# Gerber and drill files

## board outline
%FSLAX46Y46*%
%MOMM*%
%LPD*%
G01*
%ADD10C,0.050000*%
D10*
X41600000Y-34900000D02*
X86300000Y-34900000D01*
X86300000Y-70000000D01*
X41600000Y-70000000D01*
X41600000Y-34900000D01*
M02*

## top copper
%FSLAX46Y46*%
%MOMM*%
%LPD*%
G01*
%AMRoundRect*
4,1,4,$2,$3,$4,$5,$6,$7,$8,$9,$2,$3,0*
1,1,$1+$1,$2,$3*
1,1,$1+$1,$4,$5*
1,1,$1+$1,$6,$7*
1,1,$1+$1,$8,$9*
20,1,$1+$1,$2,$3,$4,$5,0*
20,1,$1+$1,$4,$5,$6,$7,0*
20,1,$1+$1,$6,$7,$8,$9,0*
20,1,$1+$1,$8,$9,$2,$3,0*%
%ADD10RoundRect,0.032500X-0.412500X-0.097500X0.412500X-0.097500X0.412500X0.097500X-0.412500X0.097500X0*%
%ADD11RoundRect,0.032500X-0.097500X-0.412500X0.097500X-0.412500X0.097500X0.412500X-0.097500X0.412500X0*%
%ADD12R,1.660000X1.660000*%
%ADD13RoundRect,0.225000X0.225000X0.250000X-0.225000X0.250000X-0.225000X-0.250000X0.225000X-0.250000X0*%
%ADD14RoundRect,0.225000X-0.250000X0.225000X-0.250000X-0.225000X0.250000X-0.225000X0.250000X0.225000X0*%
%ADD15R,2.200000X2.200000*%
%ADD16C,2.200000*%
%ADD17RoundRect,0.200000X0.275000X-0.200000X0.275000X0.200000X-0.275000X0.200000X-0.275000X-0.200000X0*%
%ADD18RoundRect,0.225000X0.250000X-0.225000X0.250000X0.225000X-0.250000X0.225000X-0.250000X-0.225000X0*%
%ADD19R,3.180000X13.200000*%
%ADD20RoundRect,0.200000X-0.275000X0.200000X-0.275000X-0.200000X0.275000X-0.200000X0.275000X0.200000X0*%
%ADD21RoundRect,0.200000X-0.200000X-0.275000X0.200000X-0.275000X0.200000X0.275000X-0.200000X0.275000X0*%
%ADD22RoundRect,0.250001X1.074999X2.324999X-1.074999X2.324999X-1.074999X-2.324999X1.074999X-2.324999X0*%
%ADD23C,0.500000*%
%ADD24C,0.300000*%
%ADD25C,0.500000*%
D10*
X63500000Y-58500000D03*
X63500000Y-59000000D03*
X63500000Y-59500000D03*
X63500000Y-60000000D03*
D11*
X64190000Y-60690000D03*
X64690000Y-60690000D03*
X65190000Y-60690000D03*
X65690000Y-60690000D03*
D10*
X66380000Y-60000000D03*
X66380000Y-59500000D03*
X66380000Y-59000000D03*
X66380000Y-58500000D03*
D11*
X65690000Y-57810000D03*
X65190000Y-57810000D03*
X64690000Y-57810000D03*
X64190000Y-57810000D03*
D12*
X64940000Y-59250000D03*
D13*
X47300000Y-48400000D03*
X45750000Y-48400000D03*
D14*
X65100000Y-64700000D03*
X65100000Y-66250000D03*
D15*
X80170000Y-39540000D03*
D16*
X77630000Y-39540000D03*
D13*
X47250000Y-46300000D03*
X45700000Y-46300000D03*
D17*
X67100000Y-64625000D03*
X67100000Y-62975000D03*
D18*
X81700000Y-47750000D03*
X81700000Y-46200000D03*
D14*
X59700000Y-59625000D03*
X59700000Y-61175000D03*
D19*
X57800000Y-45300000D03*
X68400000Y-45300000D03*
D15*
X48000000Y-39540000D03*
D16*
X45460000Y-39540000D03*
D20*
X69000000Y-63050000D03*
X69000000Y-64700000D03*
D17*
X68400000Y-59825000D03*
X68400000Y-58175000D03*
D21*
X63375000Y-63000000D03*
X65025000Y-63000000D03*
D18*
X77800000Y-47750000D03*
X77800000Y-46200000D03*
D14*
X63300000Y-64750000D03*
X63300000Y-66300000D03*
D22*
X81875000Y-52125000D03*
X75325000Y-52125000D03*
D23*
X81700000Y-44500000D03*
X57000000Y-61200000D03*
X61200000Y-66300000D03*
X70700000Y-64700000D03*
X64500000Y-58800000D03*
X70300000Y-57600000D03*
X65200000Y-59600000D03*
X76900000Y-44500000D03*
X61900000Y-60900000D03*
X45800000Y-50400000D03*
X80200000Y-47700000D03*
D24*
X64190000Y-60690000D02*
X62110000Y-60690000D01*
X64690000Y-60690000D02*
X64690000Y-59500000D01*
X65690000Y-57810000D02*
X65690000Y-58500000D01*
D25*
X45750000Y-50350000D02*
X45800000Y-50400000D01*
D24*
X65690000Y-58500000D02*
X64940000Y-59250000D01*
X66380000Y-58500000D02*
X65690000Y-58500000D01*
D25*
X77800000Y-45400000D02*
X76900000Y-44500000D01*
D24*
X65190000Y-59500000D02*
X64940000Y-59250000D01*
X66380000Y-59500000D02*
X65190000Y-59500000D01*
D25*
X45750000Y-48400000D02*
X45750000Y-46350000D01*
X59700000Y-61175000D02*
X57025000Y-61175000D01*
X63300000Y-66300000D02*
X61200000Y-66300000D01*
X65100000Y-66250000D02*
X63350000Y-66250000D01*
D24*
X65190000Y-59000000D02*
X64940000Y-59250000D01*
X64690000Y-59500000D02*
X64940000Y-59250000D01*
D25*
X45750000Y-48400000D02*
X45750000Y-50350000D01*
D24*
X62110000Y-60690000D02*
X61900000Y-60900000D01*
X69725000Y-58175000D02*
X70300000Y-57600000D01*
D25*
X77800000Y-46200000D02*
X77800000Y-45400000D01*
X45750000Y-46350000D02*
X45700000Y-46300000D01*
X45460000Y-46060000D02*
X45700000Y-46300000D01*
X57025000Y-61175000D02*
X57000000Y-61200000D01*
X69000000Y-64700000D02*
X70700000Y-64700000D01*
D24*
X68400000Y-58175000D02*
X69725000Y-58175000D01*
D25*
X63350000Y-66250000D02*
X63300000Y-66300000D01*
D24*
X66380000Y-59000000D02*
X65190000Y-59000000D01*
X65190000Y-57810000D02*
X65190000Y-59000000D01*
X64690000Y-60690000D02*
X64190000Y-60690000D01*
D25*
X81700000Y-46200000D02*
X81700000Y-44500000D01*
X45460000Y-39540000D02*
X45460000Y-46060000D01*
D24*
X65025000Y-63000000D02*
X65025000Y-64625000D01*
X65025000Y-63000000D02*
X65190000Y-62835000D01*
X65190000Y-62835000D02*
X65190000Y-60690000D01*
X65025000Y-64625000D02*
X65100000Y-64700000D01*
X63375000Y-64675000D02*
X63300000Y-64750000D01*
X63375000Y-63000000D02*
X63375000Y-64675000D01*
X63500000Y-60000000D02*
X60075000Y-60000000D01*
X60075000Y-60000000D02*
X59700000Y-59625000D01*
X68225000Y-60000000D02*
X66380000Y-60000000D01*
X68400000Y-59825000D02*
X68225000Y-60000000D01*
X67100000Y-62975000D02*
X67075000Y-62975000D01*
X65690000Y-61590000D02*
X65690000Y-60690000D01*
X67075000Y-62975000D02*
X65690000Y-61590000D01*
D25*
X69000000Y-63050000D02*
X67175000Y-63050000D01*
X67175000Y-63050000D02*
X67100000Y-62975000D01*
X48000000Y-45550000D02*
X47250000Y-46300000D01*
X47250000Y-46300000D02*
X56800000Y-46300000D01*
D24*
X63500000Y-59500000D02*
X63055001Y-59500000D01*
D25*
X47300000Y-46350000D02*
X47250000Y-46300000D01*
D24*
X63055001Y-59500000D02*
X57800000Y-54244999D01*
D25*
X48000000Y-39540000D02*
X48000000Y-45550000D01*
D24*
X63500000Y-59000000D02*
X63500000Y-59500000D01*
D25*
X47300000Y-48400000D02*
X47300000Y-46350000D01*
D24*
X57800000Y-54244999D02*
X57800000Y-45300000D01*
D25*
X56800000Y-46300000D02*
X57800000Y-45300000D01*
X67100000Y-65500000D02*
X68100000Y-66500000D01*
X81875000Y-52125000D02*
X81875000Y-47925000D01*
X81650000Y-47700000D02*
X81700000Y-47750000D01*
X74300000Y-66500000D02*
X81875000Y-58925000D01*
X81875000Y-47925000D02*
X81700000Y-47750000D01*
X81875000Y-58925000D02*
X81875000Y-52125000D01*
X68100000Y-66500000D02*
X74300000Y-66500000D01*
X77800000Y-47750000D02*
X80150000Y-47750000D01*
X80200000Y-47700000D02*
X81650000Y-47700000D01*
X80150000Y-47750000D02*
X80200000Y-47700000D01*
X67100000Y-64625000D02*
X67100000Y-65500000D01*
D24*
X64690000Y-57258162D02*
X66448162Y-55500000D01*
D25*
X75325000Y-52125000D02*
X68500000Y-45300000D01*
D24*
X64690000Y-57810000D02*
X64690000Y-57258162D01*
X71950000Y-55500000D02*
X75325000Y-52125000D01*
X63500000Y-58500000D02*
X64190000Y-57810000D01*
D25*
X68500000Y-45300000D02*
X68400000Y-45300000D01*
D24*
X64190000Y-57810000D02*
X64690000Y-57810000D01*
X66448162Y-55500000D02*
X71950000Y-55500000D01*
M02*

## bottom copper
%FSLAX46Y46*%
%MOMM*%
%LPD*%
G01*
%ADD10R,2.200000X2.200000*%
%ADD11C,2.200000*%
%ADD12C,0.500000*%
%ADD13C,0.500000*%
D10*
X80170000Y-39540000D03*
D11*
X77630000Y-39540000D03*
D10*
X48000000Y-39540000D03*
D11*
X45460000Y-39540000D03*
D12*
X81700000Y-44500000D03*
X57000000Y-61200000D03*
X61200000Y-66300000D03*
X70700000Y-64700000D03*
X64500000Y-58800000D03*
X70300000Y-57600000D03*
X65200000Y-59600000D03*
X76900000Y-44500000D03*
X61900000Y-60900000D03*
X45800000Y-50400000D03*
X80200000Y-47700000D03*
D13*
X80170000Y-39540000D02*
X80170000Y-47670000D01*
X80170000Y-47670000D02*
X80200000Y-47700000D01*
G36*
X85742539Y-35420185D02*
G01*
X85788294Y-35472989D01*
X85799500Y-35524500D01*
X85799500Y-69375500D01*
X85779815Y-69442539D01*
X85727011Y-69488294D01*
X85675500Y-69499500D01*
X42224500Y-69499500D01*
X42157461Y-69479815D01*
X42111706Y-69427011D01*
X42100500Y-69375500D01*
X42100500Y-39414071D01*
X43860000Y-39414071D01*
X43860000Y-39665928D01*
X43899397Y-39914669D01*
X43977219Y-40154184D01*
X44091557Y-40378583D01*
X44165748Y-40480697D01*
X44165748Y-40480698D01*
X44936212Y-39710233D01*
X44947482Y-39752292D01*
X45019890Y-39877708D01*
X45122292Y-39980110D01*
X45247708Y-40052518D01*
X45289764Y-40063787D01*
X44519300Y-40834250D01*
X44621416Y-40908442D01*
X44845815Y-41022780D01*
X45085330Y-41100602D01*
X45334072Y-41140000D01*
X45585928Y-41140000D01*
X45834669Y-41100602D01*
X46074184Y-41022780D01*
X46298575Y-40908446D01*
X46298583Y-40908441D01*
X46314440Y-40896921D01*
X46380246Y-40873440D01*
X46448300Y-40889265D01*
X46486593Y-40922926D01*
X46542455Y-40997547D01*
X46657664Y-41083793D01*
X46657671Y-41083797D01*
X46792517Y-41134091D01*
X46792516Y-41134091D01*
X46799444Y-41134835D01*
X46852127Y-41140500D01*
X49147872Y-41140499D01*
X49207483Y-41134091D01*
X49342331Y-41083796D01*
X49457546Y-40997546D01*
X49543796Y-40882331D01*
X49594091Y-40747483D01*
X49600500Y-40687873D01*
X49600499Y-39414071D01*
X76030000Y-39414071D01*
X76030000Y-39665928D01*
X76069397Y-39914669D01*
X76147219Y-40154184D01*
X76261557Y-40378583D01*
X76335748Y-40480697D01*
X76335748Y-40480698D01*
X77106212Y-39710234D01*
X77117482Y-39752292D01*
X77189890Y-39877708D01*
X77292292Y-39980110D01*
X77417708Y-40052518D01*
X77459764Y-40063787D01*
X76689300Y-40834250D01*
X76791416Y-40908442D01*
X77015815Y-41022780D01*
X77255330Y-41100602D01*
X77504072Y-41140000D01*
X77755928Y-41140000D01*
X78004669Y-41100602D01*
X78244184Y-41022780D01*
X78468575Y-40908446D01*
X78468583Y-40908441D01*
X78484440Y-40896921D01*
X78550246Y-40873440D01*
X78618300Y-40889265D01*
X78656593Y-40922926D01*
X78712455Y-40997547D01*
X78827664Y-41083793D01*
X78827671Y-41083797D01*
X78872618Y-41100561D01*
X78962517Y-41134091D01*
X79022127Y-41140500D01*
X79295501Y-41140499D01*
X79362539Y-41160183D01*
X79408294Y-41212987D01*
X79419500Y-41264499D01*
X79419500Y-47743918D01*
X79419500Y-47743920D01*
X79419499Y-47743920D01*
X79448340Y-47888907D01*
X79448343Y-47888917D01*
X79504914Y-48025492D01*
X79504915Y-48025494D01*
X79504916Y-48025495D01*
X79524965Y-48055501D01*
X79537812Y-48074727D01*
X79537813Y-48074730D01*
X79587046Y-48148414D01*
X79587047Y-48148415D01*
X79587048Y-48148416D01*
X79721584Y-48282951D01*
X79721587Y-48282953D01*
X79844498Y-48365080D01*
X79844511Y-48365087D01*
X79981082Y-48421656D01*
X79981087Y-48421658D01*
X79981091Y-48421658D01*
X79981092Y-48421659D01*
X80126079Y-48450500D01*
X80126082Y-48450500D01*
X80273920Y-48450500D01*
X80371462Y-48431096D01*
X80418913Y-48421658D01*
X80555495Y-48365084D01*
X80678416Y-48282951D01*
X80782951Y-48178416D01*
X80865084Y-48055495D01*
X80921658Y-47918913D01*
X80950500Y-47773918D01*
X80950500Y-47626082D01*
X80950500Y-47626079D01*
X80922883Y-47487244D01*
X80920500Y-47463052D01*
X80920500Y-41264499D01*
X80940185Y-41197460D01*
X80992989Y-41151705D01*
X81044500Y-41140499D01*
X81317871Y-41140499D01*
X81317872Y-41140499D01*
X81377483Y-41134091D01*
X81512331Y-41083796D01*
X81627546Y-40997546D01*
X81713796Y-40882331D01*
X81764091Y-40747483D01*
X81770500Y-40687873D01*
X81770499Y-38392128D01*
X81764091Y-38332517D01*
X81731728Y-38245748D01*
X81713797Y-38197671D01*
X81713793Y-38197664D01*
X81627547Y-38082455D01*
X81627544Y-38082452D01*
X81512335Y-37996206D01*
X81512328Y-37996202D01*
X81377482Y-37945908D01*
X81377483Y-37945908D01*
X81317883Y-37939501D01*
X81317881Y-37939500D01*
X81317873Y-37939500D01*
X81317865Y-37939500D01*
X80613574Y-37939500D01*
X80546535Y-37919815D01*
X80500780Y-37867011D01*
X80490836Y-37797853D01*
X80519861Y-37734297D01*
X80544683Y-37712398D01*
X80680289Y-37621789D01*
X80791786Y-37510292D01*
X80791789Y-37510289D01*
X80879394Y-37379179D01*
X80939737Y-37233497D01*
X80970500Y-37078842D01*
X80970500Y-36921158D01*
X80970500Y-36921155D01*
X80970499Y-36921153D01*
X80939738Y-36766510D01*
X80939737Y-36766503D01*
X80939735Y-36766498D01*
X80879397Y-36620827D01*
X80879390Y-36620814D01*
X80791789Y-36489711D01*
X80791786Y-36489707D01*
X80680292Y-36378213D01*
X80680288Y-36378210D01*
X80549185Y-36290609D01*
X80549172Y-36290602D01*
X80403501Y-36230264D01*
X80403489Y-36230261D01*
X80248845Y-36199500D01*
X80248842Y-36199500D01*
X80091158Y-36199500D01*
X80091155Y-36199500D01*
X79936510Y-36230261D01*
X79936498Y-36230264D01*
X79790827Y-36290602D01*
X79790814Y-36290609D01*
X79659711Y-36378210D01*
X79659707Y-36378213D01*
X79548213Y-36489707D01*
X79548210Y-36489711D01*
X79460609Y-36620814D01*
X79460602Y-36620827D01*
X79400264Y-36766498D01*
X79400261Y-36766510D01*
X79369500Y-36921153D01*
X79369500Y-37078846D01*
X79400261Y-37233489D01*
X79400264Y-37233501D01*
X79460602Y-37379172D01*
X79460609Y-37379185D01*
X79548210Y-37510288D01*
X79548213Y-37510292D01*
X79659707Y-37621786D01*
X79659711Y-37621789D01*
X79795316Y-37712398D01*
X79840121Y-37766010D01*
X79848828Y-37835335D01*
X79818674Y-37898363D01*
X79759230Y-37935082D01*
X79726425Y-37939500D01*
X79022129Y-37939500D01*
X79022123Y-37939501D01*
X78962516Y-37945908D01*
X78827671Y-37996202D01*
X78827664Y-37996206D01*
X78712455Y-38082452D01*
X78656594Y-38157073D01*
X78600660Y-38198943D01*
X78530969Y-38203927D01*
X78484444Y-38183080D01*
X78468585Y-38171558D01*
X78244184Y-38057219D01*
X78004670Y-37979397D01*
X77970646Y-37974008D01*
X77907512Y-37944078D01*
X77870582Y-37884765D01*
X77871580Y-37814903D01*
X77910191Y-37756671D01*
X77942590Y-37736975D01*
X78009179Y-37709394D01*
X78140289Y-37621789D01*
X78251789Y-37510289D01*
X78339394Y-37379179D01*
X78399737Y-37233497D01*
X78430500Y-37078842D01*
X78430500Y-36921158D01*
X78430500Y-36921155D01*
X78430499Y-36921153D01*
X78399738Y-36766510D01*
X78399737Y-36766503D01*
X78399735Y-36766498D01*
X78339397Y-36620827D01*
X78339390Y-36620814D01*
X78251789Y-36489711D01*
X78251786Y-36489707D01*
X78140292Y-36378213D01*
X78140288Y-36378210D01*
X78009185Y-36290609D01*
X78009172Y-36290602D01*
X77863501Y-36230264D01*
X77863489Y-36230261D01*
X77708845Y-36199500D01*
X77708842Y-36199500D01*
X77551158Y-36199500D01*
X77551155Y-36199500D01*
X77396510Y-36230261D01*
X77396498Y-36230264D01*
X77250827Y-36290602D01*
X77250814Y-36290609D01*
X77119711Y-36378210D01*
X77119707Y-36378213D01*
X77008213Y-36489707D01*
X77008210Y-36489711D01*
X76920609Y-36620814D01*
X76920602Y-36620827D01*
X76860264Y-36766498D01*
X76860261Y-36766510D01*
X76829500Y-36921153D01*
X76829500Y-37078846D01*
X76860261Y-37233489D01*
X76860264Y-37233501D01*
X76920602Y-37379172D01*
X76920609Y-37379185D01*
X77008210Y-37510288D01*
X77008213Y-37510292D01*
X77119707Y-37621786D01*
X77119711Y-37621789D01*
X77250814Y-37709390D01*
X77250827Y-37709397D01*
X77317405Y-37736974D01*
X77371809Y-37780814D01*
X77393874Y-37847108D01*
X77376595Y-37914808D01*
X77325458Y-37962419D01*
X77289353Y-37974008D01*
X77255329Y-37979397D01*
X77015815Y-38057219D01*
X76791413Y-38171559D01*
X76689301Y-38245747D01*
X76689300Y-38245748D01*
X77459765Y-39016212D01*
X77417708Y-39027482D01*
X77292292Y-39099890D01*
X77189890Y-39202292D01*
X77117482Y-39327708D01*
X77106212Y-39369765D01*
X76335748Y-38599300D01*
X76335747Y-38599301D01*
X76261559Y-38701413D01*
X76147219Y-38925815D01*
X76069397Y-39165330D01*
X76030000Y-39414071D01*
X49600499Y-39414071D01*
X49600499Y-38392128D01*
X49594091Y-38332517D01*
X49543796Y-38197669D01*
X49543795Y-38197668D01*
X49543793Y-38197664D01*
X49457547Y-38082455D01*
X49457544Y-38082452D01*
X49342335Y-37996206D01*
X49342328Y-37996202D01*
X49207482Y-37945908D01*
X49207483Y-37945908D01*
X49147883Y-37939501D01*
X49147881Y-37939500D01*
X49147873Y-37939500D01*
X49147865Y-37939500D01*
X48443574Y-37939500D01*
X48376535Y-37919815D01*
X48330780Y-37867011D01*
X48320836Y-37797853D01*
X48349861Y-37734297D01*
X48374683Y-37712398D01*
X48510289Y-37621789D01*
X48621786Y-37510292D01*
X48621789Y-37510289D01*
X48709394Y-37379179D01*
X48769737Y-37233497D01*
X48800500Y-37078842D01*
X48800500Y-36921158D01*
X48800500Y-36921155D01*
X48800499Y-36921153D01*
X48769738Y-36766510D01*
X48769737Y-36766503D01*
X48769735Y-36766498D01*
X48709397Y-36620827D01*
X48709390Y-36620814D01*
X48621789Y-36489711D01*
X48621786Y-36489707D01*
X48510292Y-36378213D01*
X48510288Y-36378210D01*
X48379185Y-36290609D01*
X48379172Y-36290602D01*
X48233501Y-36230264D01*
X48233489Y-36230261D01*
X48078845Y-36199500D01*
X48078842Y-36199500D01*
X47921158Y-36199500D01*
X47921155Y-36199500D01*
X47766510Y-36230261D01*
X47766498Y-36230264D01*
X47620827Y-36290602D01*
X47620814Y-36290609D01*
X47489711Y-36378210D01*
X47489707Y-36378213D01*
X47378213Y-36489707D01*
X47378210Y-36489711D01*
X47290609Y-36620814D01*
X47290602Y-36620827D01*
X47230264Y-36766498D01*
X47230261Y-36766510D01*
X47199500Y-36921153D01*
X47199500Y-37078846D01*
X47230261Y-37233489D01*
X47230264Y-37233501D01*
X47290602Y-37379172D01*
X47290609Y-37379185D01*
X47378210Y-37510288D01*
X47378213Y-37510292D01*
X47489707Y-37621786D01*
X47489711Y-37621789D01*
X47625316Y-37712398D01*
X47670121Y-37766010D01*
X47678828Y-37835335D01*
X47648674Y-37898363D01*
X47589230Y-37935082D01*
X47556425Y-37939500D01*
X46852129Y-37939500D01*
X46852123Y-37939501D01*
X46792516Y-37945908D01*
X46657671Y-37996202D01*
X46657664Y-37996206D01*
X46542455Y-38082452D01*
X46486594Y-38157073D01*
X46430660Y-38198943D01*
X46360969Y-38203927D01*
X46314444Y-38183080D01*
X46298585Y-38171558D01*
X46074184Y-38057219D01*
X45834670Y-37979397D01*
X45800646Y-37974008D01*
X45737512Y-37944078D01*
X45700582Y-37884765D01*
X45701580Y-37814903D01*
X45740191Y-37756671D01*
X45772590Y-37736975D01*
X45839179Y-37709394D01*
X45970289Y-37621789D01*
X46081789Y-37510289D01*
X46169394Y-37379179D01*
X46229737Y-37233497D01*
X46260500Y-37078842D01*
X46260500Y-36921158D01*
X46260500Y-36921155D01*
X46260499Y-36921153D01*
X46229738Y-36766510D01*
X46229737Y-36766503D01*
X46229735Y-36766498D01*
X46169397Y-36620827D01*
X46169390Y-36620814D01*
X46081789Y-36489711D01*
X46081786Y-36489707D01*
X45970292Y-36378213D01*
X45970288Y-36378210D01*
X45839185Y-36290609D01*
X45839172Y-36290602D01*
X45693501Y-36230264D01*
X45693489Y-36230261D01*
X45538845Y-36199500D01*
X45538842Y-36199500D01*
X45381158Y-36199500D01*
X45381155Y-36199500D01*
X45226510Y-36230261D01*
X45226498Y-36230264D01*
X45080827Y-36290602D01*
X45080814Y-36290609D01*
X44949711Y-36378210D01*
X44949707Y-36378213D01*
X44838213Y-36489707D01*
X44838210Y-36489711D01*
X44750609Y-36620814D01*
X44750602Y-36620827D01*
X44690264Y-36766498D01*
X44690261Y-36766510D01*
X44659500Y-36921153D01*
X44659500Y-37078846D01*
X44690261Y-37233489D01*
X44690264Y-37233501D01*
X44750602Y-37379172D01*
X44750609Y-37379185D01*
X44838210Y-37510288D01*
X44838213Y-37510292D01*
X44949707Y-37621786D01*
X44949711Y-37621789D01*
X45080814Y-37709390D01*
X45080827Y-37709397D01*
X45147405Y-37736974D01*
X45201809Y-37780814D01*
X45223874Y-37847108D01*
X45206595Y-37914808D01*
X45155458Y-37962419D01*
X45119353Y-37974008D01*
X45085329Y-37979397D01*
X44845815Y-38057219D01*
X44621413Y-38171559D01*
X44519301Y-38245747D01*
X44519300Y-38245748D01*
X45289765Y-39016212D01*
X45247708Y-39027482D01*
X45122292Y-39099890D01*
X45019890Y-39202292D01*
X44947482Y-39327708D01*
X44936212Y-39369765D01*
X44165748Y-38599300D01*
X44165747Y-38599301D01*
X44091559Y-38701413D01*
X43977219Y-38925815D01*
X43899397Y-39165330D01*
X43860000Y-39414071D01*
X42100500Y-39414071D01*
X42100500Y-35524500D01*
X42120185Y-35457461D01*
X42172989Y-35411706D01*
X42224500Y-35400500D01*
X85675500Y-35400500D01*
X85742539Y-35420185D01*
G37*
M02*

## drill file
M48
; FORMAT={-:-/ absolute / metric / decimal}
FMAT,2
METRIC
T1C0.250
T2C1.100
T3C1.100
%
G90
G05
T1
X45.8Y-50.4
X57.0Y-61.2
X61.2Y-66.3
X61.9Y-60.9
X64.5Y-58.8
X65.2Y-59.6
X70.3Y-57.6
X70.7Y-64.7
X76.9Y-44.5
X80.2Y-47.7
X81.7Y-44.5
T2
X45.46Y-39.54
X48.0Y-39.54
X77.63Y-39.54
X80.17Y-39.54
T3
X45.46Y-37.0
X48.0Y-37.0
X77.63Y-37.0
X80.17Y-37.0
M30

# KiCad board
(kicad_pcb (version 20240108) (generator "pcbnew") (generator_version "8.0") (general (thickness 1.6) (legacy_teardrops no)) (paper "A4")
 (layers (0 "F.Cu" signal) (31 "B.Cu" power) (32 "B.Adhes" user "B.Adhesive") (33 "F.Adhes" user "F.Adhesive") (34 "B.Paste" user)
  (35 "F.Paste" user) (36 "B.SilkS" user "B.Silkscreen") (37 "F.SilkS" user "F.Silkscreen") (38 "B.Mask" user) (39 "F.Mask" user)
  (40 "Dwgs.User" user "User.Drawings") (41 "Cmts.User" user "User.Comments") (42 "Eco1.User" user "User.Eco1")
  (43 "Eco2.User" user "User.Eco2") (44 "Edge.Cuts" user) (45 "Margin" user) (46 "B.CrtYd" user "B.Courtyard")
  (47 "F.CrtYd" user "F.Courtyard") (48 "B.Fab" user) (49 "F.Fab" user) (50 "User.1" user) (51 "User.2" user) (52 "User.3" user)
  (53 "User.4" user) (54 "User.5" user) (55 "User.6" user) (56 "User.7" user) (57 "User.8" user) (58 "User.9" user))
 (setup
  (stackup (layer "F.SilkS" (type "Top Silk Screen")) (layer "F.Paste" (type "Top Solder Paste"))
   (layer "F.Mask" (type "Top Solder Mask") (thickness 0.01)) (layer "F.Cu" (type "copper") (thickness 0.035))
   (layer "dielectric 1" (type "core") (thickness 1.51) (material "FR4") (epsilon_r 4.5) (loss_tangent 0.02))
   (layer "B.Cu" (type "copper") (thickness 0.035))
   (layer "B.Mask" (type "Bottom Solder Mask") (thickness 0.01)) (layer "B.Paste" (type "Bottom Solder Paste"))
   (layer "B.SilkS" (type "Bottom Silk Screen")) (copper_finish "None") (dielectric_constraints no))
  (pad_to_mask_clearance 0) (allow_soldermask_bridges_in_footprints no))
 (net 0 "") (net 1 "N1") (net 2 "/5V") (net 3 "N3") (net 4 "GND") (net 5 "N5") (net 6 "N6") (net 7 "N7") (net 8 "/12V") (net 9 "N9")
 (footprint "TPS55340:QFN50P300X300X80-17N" (layer "F.Cu") (at 64.94 59.25)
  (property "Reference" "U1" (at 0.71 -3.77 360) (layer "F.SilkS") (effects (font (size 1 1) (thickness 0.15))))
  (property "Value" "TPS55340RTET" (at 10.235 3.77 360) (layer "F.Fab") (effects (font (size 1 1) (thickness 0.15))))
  (pad "1" smd roundrect (at -1.44 -0.75) (size 0.89 0.26) (layers "F.Cu" "F.Paste" "F.Mask") (roundrect_rratio 0.125) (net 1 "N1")
   (solder_mask_margin 0.102))
  (pad "2" smd roundrect (at -1.44 -0.25) (size 0.89 0.26) (layers "F.Cu" "F.Paste" "F.Mask") (roundrect_rratio 0.125) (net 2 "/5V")
   (solder_mask_margin 0.102))
  (pad "3" smd roundrect (at -1.44 0.25) (size 0.89 0.26) (layers "F.Cu" "F.Paste" "F.Mask") (roundrect_rratio 0.125) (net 2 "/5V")
   (solder_mask_margin 0.102))
  (pad "4" smd roundrect (at -1.44 0.75) (size 0.89 0.26) (layers "F.Cu" "F.Paste" "F.Mask") (roundrect_rratio 0.125) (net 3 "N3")
   (solder_mask_margin 0.102))
  (pad "5" smd roundrect (at -0.75 1.44) (size 0.26 0.89) (layers "F.Cu" "F.Paste" "F.Mask") (roundrect_rratio 0.125) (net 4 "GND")
   (solder_mask_margin 0.102))
  (pad "6" smd roundrect (at -0.25 1.44) (size 0.26 0.89) (layers "F.Cu" "F.Paste" "F.Mask") (roundrect_rratio 0.125) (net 4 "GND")
   (solder_mask_margin 0.102))
  (pad "7" smd roundrect (at 0.25 1.44) (size 0.26 0.89) (layers "F.Cu" "F.Paste" "F.Mask") (roundrect_rratio 0.125) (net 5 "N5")
   (solder_mask_margin 0.102))
  (pad "8" smd roundrect (at 0.75 1.44) (size 0.26 0.89) (layers "F.Cu" "F.Paste" "F.Mask") (roundrect_rratio 0.125) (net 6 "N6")
   (solder_mask_margin 0.102))
  (pad "9" smd roundrect (at 1.44 0.75) (size 0.89 0.26) (layers "F.Cu" "F.Paste" "F.Mask") (roundrect_rratio 0.125) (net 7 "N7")
   (solder_mask_margin 0.102))
  (pad "10" smd roundrect (at 1.44 0.25) (size 0.89 0.26) (layers "F.Cu" "F.Paste" "F.Mask") (roundrect_rratio 0.125) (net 4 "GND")
   (solder_mask_margin 0.102))
  (pad "11" smd roundrect (at 1.44 -0.25) (size 0.89 0.26) (layers "F.Cu" "F.Paste" "F.Mask") (roundrect_rratio 0.125) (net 4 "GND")
   (solder_mask_margin 0.102))
  (pad "12" smd roundrect (at 1.44 -0.75) (size 0.89 0.26) (layers "F.Cu" "F.Paste" "F.Mask") (roundrect_rratio 0.125) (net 4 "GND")
   (solder_mask_margin 0.102))
  (pad "13" smd roundrect (at 0.75 -1.44) (size 0.26 0.89) (layers "F.Cu" "F.Paste" "F.Mask") (roundrect_rratio 0.125) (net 4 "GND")
   (solder_mask_margin 0.102))
  (pad "14" smd roundrect (at 0.25 -1.44) (size 0.26 0.89) (layers "F.Cu" "F.Paste" "F.Mask") (roundrect_rratio 0.125) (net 4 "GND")
   (solder_mask_margin 0.102))
  (pad "15" smd roundrect (at -0.25 -1.44) (size 0.26 0.89) (layers "F.Cu" "F.Paste" "F.Mask") (roundrect_rratio 0.125) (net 1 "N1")
   (solder_mask_margin 0.102))
  (pad "16" smd roundrect (at -0.75 -1.44) (size 0.26 0.89) (layers "F.Cu" "F.Paste" "F.Mask") (roundrect_rratio 0.125) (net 1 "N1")
   (solder_mask_margin 0.102))
  (pad "17" smd rect (at 0 0) (size 1.66 1.66) (layers "F.Cu" "F.Mask") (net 4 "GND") (solder_mask_margin 0.102)))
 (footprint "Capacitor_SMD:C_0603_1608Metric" (layer "F.Cu") (at 46.525 48.4 180)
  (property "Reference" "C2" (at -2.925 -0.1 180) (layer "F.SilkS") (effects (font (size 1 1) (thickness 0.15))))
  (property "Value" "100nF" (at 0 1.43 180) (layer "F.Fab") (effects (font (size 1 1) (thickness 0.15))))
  (pad "1" smd roundrect (at -0.775 0 180) (size 0.9 0.95) (layers "F.Cu" "F.Paste" "F.Mask") (roundrect_rratio 0.25) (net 2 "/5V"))
  (pad "2" smd roundrect (at 0.775 0 180) (size 0.9 0.95) (layers "F.Cu" "F.Paste" "F.Mask") (roundrect_rratio 0.25) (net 4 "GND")))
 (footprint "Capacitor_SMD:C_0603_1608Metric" (layer "F.Cu") (at 65.1 65.475 -90)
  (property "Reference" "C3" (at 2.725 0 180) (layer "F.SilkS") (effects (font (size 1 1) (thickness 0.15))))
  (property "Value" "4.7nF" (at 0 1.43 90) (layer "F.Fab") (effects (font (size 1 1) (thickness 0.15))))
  (pad "1" smd roundrect (at -0.775 0 270) (size 0.9 0.95) (layers "F.Cu" "F.Paste" "F.Mask") (roundrect_rratio 0.25) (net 5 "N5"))
  (pad "2" smd roundrect (at 0.775 0 270) (size 0.9 0.95) (layers "F.Cu" "F.Paste" "F.Mask") (roundrect_rratio 0.25) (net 4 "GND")))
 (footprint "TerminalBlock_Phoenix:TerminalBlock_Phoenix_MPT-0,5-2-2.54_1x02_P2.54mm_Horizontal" (layer "F.Cu") (at 80.17 39.54 180)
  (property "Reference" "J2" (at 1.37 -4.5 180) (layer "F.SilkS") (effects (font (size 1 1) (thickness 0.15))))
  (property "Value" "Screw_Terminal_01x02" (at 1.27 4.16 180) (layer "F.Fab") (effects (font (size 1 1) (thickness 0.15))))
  (pad "" np_thru_hole circle (at 0 2.54 180) (size 1.1 1.1) (drill 1.1) (layers "*.Cu" "*.Mask"))
  (pad "" np_thru_hole circle (at 2.54 2.54 180) (size 1.1 1.1) (drill 1.1) (layers "*.Cu" "*.Mask"))
  (pad "1" thru_hole rect (at 0 0 180) (size 2.2 2.2) (drill 1.1) (layers "*.Cu" "*.Mask") (remove_unused_layers no) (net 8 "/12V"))
  (pad "2" thru_hole circle (at 2.54 0 180) (size 2.2 2.2) (drill 1.1) (layers "*.Cu" "*.Mask") (remove_unused_layers no) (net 4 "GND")))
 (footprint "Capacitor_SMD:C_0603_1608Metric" (layer "F.Cu") (at 46.475 46.3 180)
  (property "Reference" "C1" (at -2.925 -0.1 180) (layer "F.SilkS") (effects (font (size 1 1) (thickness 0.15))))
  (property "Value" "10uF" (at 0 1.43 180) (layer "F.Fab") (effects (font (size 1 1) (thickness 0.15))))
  (pad "1" smd roundrect (at -0.775 0 180) (size 0.9 0.95) (layers "F.Cu" "F.Paste" "F.Mask") (roundrect_rratio 0.25) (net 2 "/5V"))
  (pad "2" smd roundrect (at 0.775 0 180) (size 0.9 0.95) (layers "F.Cu" "F.Paste" "F.Mask") (roundrect_rratio 0.25) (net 4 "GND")))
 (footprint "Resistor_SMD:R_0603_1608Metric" (layer "F.Cu") (at 67.1 63.8 90)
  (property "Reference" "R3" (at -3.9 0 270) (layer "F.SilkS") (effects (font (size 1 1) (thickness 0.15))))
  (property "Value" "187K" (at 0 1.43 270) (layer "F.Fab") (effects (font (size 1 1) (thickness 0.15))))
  (pad "1" smd roundrect (at -0.825 0 90) (size 0.8 0.95) (layers "F.Cu" "F.Paste" "F.Mask") (roundrect_rratio 0.25) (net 8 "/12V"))
  (pad "2" smd roundrect (at 0.825 0 90) (size 0.8 0.95) (layers "F.Cu" "F.Paste" "F.Mask") (roundrect_rratio 0.25) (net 6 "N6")))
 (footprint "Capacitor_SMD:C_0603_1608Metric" (layer "F.Cu") (at 81.7 46.975 90)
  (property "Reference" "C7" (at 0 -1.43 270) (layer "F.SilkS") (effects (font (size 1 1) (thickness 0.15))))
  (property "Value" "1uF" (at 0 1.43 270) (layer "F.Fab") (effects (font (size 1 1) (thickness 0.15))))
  (pad "1" smd roundrect (at -0.775 0 90) (size 0.9 0.95) (layers "F.Cu" "F.Paste" "F.Mask") (roundrect_rratio 0.25) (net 8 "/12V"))
  (pad "2" smd roundrect (at 0.775 0 90) (size 0.9 0.95) (layers "F.Cu" "F.Paste" "F.Mask") (roundrect_rratio 0.25) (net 4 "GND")))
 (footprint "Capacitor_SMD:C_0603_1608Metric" (layer "F.Cu") (at 59.7 60.4 -90)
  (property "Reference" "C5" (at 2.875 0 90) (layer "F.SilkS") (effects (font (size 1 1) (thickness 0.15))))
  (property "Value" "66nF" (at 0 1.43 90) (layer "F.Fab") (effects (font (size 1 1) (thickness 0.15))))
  (pad "1" smd roundrect (at -0.775 0 270) (size 0.9 0.95) (layers "F.Cu" "F.Paste" "F.Mask") (roundrect_rratio 0.25) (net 3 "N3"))
  (pad "2" smd roundrect (at 0.775 0 270) (size 0.9 0.95) (layers "F.Cu" "F.Paste" "F.Mask") (roundrect_rratio 0.25) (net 4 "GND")))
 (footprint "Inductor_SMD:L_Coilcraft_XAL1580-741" (layer "F.Cu") (at 63.1 45.3)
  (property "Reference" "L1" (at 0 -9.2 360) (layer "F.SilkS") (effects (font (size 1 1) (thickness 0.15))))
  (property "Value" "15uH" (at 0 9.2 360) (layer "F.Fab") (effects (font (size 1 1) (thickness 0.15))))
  (pad "1" smd rect (at -5.3 0) (size 3.18 13.2) (layers "F.Cu" "F.Paste" "F.Mask") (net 2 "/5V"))
  (pad "2" smd rect (at 5.3 0) (size 3.18 13.2) (layers "F.Cu" "F.Paste" "F.Mask") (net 1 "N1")))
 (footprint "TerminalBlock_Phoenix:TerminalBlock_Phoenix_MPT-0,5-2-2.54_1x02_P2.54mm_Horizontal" (layer "F.Cu") (at 48 39.54 180)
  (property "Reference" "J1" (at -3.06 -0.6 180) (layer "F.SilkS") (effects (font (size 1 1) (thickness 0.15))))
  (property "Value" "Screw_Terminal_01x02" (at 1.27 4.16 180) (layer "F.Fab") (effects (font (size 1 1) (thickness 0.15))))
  (pad "" np_thru_hole circle (at 0 2.54 180) (size 1.1 1.1) (drill 1.1) (layers "*.Cu" "*.Mask"))
  (pad "" np_thru_hole circle (at 2.54 2.54 180) (size 1.1 1.1) (drill 1.1) (layers "*.Cu" "*.Mask"))
  (pad "1" thru_hole rect (at 0 0 180) (size 2.2 2.2) (drill 1.1) (layers "*.Cu" "*.Mask") (remove_unused_layers no) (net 2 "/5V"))
  (pad "2" thru_hole circle (at 2.54 0 180) (size 2.2 2.2) (drill 1.1) (layers "*.Cu" "*.Mask") (remove_unused_layers no) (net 4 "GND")))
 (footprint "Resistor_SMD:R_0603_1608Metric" (layer "F.Cu") (at 69 63.875 -90)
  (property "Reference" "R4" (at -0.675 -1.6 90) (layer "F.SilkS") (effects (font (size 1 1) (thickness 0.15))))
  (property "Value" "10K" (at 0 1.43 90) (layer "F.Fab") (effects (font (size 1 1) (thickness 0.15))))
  (pad "1" smd roundrect (at -0.825 0 270) (size 0.8 0.95) (layers "F.Cu" "F.Paste" "F.Mask") (roundrect_rratio 0.25) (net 6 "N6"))
  (pad "2" smd roundrect (at 0.825 0 270) (size 0.8 0.95) (layers "F.Cu" "F.Paste" "F.Mask") (roundrect_rratio 0.25) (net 4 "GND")))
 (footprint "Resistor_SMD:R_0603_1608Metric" (layer "F.Cu") (at 68.4 59 90)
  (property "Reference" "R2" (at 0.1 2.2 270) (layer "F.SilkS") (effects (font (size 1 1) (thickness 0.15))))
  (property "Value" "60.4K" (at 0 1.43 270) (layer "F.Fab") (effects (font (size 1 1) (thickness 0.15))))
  (pad "1" smd roundrect (at -0.825 0 90) (size 0.8 0.95) (layers "F.Cu" "F.Paste" "F.Mask") (roundrect_rratio 0.25) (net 7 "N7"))
  (pad "2" smd roundrect (at 0.825 0 90) (size 0.8 0.95) (layers "F.Cu" "F.Paste" "F.Mask") (roundrect_rratio 0.25) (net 4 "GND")))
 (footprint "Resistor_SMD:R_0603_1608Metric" (layer "F.Cu") (at 64.2 63)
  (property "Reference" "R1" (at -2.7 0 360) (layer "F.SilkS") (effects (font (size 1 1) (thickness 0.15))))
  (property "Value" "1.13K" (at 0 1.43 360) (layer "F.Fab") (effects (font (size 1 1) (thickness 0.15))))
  (pad "1" smd roundrect (at -0.825 0) (size 0.8 0.95) (layers "F.Cu" "F.Paste" "F.Mask") (roundrect_rratio 0.25) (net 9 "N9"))
  (pad "2" smd roundrect (at 0.825 0) (size 0.8 0.95) (layers "F.Cu" "F.Paste" "F.Mask") (roundrect_rratio 0.25) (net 5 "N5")))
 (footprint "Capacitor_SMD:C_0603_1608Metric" (layer "F.Cu") (at 77.8 46.975 90)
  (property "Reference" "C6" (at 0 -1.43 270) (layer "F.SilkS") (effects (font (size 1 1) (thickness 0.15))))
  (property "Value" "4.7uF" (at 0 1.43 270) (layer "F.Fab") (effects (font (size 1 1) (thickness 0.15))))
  (pad "1" smd roundrect (at -0.775 0 90) (size 0.9 0.95) (layers "F.Cu" "F.Paste" "F.Mask") (roundrect_rratio 0.25) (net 8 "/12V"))
  (pad "2" smd roundrect (at 0.775 0 90) (size 0.9 0.95) (layers "F.Cu" "F.Paste" "F.Mask") (roundrect_rratio 0.25) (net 4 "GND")))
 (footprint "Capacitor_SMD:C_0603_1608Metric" (layer "F.Cu") (at 63.3 65.525 -90)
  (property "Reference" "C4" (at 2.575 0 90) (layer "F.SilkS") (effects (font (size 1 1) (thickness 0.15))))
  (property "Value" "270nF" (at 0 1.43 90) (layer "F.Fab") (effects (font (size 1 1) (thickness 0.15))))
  (pad "1" smd roundrect (at -0.775 0 270) (size 0.9 0.95) (layers "F.Cu" "F.Paste" "F.Mask") (roundrect_rratio 0.25) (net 9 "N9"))
  (pad "2" smd roundrect (at 0.775 0 270) (size 0.9 0.95) (layers "F.Cu" "F.Paste" "F.Mask") (roundrect_rratio 0.25) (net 4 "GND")))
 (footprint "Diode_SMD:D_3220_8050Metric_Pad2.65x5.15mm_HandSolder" (layer "F.Cu") (at 78.6 52.125 180)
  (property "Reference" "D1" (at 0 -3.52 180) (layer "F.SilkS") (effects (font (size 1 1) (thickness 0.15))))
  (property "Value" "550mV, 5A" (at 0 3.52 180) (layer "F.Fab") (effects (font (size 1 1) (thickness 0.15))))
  (pad "1" smd roundrect (at -3.275 0 180) (size 2.65 5.15) (layers "F.Cu" "F.Paste" "F.Mask") (roundrect_rratio 0.09434) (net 8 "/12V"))
  (pad "2" smd roundrect (at 3.275 0 180) (size 2.65 5.15) (layers "F.Cu" "F.Paste" "F.Mask") (roundrect_rratio 0.09434) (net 1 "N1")))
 (gr_rect (start 41.6 34.9) (end 86.3 70) (stroke (width 0.05) (type default)) (fill none) (layer "Edge.Cuts"))
 (segment (start 64.19 60.69) (end 62.11 60.69) (width 0.3) (layer "F.Cu") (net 4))
 (segment (start 64.69 60.69) (end 64.69 59.5) (width 0.3) (layer "F.Cu") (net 4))
 (segment (start 65.69 57.81) (end 65.69 58.5) (width 0.3) (layer "F.Cu") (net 4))
 (segment (start 45.75 50.35) (end 45.8 50.4) (width 0.5) (layer "F.Cu") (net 4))
 (segment (start 65.69 58.5) (end 64.94 59.25) (width 0.3) (layer "F.Cu") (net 4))
 (segment (start 66.38 58.5) (end 65.69 58.5) (width 0.3) (layer "F.Cu") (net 4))
 (segment (start 77.8 45.4) (end 76.9 44.5) (width 0.5) (layer "F.Cu") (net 4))
 (segment (start 65.19 59.5) (end 64.94 59.25) (width 0.3) (layer "F.Cu") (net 4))
 (segment (start 66.38 59.5) (end 65.19 59.5) (width 0.3) (layer "F.Cu") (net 4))
 (segment (start 45.75 48.4) (end 45.75 46.35) (width 0.5) (layer "F.Cu") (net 4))
 (segment (start 59.7 61.175) (end 57.025 61.175) (width 0.5) (layer "F.Cu") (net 4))
 (segment (start 63.3 66.3) (end 61.2 66.3) (width 0.5) (layer "F.Cu") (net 4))
 (segment (start 65.1 66.25) (end 63.35 66.25) (width 0.5) (layer "F.Cu") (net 4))
 (segment (start 65.19 59) (end 64.94 59.25) (width 0.3) (layer "F.Cu") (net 4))
 (segment (start 64.69 59.5) (end 64.94 59.25) (width 0.3) (layer "F.Cu") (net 4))
 (segment (start 45.75 48.4) (end 45.75 50.35) (width 0.5) (layer "F.Cu") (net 4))
 (segment (start 62.11 60.69) (end 61.9 60.9) (width 0.3) (layer "F.Cu") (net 4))
 (segment (start 69.725 58.175) (end 70.3 57.6) (width 0.3) (layer "F.Cu") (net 4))
 (segment (start 77.8 46.2) (end 77.8 45.4) (width 0.5) (layer "F.Cu") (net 4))
 (segment (start 45.75 46.35) (end 45.7 46.3) (width 0.5) (layer "F.Cu") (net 4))
 (segment (start 45.46 46.06) (end 45.7 46.3) (width 0.5) (layer "F.Cu") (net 4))
 (segment (start 57.025 61.175) (end 57 61.2) (width 0.5) (layer "F.Cu") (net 4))
 (segment (start 69 64.7) (end 70.7 64.7) (width 0.5) (layer "F.Cu") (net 4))
 (segment (start 68.4 58.175) (end 69.725 58.175) (width 0.3) (layer "F.Cu") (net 4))
 (segment (start 63.35 66.25) (end 63.3 66.3) (width 0.5) (layer "F.Cu") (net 4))
 (segment (start 66.38 59) (end 65.19 59) (width 0.3) (layer "F.Cu") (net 4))
 (segment (start 65.19 57.81) (end 65.19 59) (width 0.3) (layer "F.Cu") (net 4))
 (segment (start 64.69 60.69) (end 64.19 60.69) (width 0.3) (layer "F.Cu") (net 4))
 (segment (start 81.7 46.2) (end 81.7 44.5) (width 0.5) (layer "F.Cu") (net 4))
 (segment (start 45.46 39.54) (end 45.46 46.06) (width 0.5) (layer "F.Cu") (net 4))
 (via (at 81.7 44.5) (size 0.5) (drill 0.25) (layers "F.Cu" "B.Cu") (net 4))
 (via (at 57 61.2) (size 0.5) (drill 0.25) (layers "F.Cu" "B.Cu") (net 4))
 (via (at 61.2 66.3) (size 0.5) (drill 0.25) (layers "F.Cu" "B.Cu") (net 4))
 (via (at 70.7 64.7) (size 0.5) (drill 0.25) (layers "F.Cu" "B.Cu") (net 4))
 (via (at 64.5 58.8) (size 0.5) (drill 0.25) (layers "F.Cu" "B.Cu") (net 4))
 (via (at 70.3 57.6) (size 0.5) (drill 0.25) (layers "F.Cu" "B.Cu") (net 4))
 (via (at 65.2 59.6) (size 0.5) (drill 0.25) (layers "F.Cu" "B.Cu") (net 4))
 (via (at 76.9 44.5) (size 0.5) (drill 0.25) (layers "F.Cu" "B.Cu") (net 4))
 (via (at 61.9 60.9) (size 0.5) (drill 0.25) (layers "F.Cu" "B.Cu") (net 4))
 (via (at 45.8 50.4) (size 0.5) (drill 0.25) (layers "F.Cu" "B.Cu") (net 4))
 (segment (start 65.025 63) (end 65.025 64.625) (width 0.3) (layer "F.Cu") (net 5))
 (segment (start 65.025 63) (end 65.19 62.835) (width 0.3) (layer "F.Cu") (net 5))
 (segment (start 65.19 62.835) (end 65.19 60.69) (width 0.3) (layer "F.Cu") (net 5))
 (segment (start 65.025 64.625) (end 65.1 64.7) (width 0.3) (layer "F.Cu") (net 5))
 (segment (start 63.375 64.675) (end 63.3 64.75) (width 0.3) (layer "F.Cu") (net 9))
 (segment (start 63.375 63) (end 63.375 64.675) (width 0.3) (layer "F.Cu") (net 9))
 (segment (start 63.5 60) (end 60.075 60) (width 0.3) (layer "F.Cu") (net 3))
 (segment (start 60.075 60) (end 59.7 59.625) (width 0.3) (layer "F.Cu") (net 3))
 (segment (start 68.225 60) (end 66.38 60) (width 0.3) (layer "F.Cu") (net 7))
 (segment (start 68.4 59.825) (end 68.225 60) (width 0.3) (layer "F.Cu") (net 7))
 (segment (start 67.1 62.975) (end 67.075 62.975) (width 0.3) (layer "F.Cu") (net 6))
 (segment (start 65.69 61.59) (end 65.69 60.69) (width 0.3) (layer "F.Cu") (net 6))
 (segment (start 67.075 62.975) (end 65.69 61.59) (width 0.3) (layer "F.Cu") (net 6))
 (segment (start 69 63.05) (end 67.175 63.05) (width 0.5) (layer "F.Cu") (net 6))
 (segment (start 67.175 63.05) (end 67.1 62.975) (width 0.5) (layer "F.Cu") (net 6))
 (segment (start 48 45.55) (end 47.25 46.3) (width 0.5) (layer "F.Cu") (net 2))
 (segment (start 47.25 46.3) (end 56.8 46.3) (width 0.5) (layer "F.Cu") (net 2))
 (segment (start 63.5 59.5) (end 63.055001 59.5) (width 0.3) (layer "F.Cu") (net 2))
 (segment (start 47.3 46.35) (end 47.25 46.3) (width 0.5) (layer "F.Cu") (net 2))
 (segment (start 63.055001 59.5) (end 57.8 54.244999) (width 0.3) (layer "F.Cu") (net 2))
 (segment (start 48 39.54) (end 48 45.55) (width 0.5) (layer "F.Cu") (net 2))
 (segment (start 63.5 59) (end 63.5 59.5) (width 0.3) (layer "F.Cu") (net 2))
 (segment (start 47.3 48.4) (end 47.3 46.35) (width 0.5) (layer "F.Cu") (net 2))
 (segment (start 57.8 54.244999) (end 57.8 45.3) (width 0.3) (layer "F.Cu") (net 2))
 (segment (start 56.8 46.3) (end 57.8 45.3) (width 0.5) (layer "F.Cu") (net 2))
 (segment (start 67.1 65.5) (end 68.1 66.5) (width 0.5) (layer "F.Cu") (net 8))
 (segment (start 81.875 52.125) (end 81.875 47.925) (width 0.5) (layer "F.Cu") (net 8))
 (segment (start 81.65 47.7) (end 81.7 47.75) (width 0.5) (layer "F.Cu") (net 8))
 (segment (start 74.3 66.5) (end 81.875 58.925) (width 0.5) (layer "F.Cu") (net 8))
 (segment (start 81.875 47.925) (end 81.7 47.75) (width 0.5) (layer "F.Cu") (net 8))
 (segment (start 81.875 58.925) (end 81.875 52.125) (width 0.5) (layer "F.Cu") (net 8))
 (segment (start 68.1 66.5) (end 74.3 66.5) (width 0.5) (layer "F.Cu") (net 8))
 (segment (start 77.8 47.75) (end 80.15 47.75) (width 0.5) (layer "F.Cu") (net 8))
 (segment (start 80.2 47.7) (end 81.65 47.7) (width 0.5) (layer "F.Cu") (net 8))
 (segment (start 80.15 47.75) (end 80.2 47.7) (width 0.5) (layer "F.Cu") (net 8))
 (segment (start 67.1 64.625) (end 67.1 65.5) (width 0.5) (layer "F.Cu") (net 8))
 (via (at 80.2 47.7) (size 0.5) (drill 0.25) (layers "F.Cu" "B.Cu") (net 8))
 (segment (start 80.17 39.54) (end 80.17 47.67) (width 0.5) (layer "B.Cu") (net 8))
 (segment (start 80.17 47.67) (end 80.2 47.7) (width 0.5) (layer "B.Cu") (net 8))
 (segment (start 64.69 57.258162) (end 66.448162 55.5) (width 0.3) (layer "F.Cu") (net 1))
 (segment (start 75.325 52.125) (end 68.5 45.3) (width 0.5) (layer "F.Cu") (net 1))
 (segment (start 64.69 57.81) (end 64.69 57.258162) (width 0.3) (layer "F.Cu") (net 1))
 (segment (start 71.95 55.5) (end 75.325 52.125) (width 0.3) (layer "F.Cu") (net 1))
 (segment (start 63.5 58.5) (end 64.19 57.81) (width 0.3) (layer "F.Cu") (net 1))
 (segment (start 68.5 45.3) (end 68.4 45.3) (width 0.5) (layer "F.Cu") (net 1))
 (segment (start 64.19 57.81) (end 64.69 57.81) (width 0.3) (layer "F.Cu") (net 1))
 (segment (start 66.448162 55.5) (end 71.95 55.5) (width 0.3) (layer "F.Cu") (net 1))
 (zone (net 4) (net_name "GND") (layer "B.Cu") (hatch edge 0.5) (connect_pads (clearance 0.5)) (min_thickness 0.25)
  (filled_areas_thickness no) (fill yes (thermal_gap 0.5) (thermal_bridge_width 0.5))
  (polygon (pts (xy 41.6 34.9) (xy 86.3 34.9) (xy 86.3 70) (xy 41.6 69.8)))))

